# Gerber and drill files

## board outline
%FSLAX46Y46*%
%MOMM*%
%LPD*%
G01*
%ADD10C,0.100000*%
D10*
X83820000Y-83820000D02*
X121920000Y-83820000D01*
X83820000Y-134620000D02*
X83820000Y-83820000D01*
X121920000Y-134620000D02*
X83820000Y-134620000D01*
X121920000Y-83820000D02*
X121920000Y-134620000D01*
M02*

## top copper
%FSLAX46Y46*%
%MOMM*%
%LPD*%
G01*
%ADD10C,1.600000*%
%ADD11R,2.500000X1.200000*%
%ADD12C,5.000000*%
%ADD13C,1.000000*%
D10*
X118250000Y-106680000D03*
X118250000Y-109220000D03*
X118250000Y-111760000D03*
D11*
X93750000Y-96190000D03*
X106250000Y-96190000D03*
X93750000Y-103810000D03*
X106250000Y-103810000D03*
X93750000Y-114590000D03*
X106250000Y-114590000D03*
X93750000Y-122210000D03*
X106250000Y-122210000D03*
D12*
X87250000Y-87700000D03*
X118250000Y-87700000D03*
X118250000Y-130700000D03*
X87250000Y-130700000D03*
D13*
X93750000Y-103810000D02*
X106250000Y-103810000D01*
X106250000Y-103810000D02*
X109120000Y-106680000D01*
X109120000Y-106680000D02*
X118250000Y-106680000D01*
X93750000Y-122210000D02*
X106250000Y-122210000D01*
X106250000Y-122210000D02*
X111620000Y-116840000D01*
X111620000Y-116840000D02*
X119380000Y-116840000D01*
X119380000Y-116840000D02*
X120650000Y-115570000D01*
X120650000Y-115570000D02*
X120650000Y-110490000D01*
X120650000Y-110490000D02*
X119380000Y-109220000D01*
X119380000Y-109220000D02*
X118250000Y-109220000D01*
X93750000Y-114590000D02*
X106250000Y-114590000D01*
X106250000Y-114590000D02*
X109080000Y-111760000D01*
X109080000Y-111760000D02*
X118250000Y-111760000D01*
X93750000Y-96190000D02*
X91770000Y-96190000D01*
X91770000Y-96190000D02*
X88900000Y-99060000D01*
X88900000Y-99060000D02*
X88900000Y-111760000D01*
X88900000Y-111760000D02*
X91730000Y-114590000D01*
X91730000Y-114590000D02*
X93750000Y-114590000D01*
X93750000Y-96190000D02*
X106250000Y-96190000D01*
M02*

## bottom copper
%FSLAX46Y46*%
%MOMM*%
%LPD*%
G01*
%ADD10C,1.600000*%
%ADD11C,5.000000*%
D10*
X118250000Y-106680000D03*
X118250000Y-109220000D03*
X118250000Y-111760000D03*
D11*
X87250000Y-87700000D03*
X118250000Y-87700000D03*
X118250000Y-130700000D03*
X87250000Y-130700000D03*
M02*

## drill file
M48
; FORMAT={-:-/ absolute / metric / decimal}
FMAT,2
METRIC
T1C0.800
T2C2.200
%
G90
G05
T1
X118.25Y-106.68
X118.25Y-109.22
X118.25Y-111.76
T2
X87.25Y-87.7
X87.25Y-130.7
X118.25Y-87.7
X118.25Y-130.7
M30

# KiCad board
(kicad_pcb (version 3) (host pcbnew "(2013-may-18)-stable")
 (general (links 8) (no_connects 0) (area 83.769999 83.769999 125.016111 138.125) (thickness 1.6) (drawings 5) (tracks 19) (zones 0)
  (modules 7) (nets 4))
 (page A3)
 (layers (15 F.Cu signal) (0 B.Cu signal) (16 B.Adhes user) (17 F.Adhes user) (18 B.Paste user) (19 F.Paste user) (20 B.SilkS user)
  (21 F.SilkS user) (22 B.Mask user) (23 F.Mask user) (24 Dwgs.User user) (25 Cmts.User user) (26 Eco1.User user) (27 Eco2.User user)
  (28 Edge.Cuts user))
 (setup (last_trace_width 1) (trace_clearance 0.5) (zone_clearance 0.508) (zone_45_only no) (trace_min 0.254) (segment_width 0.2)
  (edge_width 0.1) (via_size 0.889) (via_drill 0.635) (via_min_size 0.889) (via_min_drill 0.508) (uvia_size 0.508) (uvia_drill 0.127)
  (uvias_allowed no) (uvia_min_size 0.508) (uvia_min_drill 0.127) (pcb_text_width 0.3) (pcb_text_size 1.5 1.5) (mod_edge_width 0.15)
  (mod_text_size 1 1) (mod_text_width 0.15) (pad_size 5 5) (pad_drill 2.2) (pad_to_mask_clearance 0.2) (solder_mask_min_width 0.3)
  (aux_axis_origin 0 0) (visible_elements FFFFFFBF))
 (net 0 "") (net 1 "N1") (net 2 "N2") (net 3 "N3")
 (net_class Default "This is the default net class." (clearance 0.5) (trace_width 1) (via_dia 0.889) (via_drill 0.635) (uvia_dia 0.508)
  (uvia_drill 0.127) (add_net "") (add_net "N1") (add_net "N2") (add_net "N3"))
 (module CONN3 (layer F.Cu) (at 118.25 109.22 270)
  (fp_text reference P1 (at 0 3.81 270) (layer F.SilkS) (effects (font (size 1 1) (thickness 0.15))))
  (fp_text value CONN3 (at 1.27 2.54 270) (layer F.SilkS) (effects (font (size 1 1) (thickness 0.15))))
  (pad 1 thru_hole circle (at -2.54 0 270) (size 1.6 1.6) (drill 0.8) (layers *.Cu *.Mask F.SilkS) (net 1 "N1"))
  (pad 2 thru_hole circle (at 0 0 270) (size 1.6 1.6) (drill 0.8) (layers *.Cu *.Mask F.SilkS) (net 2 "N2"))
  (pad 3 thru_hole circle (at 2.54 0 270) (size 1.6 1.6) (drill 0.8) (layers *.Cu *.Mask F.SilkS) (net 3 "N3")))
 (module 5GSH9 (layer F.Cu) (at 100 100)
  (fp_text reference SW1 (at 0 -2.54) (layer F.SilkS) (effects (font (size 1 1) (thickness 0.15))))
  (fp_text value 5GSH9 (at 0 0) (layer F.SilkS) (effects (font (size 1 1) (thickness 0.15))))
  (pad 2 smd rect (at -6.25 -3.81) (size 2.5 1.2) (layers F.Cu F.Paste F.Mask) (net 3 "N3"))
  (pad 1 smd rect (at 6.25 -3.81) (size 2.5 1.2) (layers F.Cu F.Paste F.Mask) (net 3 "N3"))
  (pad 4 smd rect (at -6.25 3.81) (size 2.5 1.2) (layers F.Cu F.Paste F.Mask) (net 1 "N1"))
  (pad 3 smd rect (at 6.25 3.81) (size 2.5 1.2) (layers F.Cu F.Paste F.Mask) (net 1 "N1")))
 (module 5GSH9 (layer F.Cu) (at 100 118.4)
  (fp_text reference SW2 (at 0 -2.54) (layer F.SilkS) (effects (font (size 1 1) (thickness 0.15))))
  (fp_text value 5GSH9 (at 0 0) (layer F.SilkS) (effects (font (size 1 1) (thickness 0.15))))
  (pad 2 smd rect (at -6.25 -3.81) (size 2.5 1.2) (layers F.Cu F.Paste F.Mask) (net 3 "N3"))
  (pad 1 smd rect (at 6.25 -3.81) (size 2.5 1.2) (layers F.Cu F.Paste F.Mask) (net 3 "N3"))
  (pad 4 smd rect (at -6.25 3.81) (size 2.5 1.2) (layers F.Cu F.Paste F.Mask) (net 2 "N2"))
  (pad 3 smd rect (at 6.25 3.81) (size 2.5 1.2) (layers F.Cu F.Paste F.Mask) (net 2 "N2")))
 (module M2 (layer F.Cu) (at 87.25 87.7)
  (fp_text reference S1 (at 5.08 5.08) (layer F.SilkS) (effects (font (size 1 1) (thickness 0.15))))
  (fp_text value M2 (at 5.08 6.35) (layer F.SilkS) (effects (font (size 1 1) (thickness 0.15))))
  (pad P thru_hole circle (at 0 0) (size 5 5) (drill 2.2) (layers *.Cu *.Mask F.SilkS)))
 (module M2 (layer F.Cu) (at 118.25 87.7)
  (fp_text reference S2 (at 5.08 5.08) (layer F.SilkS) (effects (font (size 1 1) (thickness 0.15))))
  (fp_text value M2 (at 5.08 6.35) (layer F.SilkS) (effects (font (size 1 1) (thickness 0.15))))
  (pad P thru_hole circle (at 0 0) (size 5 5) (drill 2.2) (layers *.Cu *.Mask F.SilkS)))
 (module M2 (layer F.Cu) (at 118.25 130.7)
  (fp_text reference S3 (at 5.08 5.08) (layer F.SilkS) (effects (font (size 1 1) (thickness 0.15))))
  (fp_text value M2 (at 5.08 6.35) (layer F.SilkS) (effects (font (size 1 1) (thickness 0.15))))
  (pad P thru_hole circle (at 0 0) (size 5 5) (drill 2.2) (layers *.Cu *.Mask F.SilkS)))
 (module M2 (layer F.Cu) (at 87.25 130.7)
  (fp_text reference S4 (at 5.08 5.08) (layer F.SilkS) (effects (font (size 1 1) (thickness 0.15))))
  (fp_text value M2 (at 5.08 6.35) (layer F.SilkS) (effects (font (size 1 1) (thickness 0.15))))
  (pad P thru_hole circle (at 0 0) (size 5 5) (drill 2.2) (layers *.Cu *.Mask F.SilkS)))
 (gr_line (start 83.82 83.82) (end 121.92 83.82) (angle 90) (layer Edge.Cuts) (width 0.1))
 (gr_line (start 83.82 134.62) (end 83.82 83.82) (angle 90) (layer Edge.Cuts) (width 0.1))
 (gr_line (start 121.92 134.62) (end 83.82 134.62) (angle 90) (layer Edge.Cuts) (width 0.1))
 (gr_line (start 121.92 83.82) (end 121.92 134.62) (angle 90) (layer Edge.Cuts) (width 0.1))
 (segment (start 93.75 103.81) (end 106.25 103.81) (width 1) (layer F.Cu) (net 1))
 (segment (start 106.25 103.81) (end 109.12 106.68) (width 1) (layer F.Cu) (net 1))
 (segment (start 109.12 106.68) (end 118.25 106.68) (width 1) (layer F.Cu) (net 1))
 (segment (start 93.75 122.21) (end 106.25 122.21) (width 1) (layer F.Cu) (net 2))
 (segment (start 106.25 122.21) (end 111.62 116.84) (width 1) (layer F.Cu) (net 2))
 (segment (start 111.62 116.84) (end 119.38 116.84) (width 1) (layer F.Cu) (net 2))
 (segment (start 119.38 116.84) (end 120.65 115.57) (width 1) (layer F.Cu) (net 2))
 (segment (start 120.65 115.57) (end 120.65 110.49) (width 1) (layer F.Cu) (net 2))
 (segment (start 120.65 110.49) (end 119.38 109.22) (width 1) (layer F.Cu) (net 2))
 (segment (start 119.38 109.22) (end 118.25 109.22) (width 1) (layer F.Cu) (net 2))
 (segment (start 93.75 114.59) (end 106.25 114.59) (width 1) (layer F.Cu) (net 3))
 (segment (start 106.25 114.59) (end 109.08 111.76) (width 1) (layer F.Cu) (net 3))
 (segment (start 109.08 111.76) (end 118.25 111.76) (width 1) (layer F.Cu) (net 3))
 (segment (start 93.75 96.19) (end 91.77 96.19) (width 1) (layer F.Cu) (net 3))
 (segment (start 91.77 96.19) (end 88.9 99.06) (width 1) (layer F.Cu) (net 3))
 (segment (start 88.9 99.06) (end 88.9 111.76) (width 1) (layer F.Cu) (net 3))
 (segment (start 88.9 111.76) (end 91.73 114.59) (width 1) (layer F.Cu) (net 3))
 (segment (start 91.73 114.59) (end 93.75 114.59) (width 1) (layer F.Cu) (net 3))
 (segment (start 93.75 96.19) (end 106.25 96.19) (width 1) (layer F.Cu) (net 3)))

